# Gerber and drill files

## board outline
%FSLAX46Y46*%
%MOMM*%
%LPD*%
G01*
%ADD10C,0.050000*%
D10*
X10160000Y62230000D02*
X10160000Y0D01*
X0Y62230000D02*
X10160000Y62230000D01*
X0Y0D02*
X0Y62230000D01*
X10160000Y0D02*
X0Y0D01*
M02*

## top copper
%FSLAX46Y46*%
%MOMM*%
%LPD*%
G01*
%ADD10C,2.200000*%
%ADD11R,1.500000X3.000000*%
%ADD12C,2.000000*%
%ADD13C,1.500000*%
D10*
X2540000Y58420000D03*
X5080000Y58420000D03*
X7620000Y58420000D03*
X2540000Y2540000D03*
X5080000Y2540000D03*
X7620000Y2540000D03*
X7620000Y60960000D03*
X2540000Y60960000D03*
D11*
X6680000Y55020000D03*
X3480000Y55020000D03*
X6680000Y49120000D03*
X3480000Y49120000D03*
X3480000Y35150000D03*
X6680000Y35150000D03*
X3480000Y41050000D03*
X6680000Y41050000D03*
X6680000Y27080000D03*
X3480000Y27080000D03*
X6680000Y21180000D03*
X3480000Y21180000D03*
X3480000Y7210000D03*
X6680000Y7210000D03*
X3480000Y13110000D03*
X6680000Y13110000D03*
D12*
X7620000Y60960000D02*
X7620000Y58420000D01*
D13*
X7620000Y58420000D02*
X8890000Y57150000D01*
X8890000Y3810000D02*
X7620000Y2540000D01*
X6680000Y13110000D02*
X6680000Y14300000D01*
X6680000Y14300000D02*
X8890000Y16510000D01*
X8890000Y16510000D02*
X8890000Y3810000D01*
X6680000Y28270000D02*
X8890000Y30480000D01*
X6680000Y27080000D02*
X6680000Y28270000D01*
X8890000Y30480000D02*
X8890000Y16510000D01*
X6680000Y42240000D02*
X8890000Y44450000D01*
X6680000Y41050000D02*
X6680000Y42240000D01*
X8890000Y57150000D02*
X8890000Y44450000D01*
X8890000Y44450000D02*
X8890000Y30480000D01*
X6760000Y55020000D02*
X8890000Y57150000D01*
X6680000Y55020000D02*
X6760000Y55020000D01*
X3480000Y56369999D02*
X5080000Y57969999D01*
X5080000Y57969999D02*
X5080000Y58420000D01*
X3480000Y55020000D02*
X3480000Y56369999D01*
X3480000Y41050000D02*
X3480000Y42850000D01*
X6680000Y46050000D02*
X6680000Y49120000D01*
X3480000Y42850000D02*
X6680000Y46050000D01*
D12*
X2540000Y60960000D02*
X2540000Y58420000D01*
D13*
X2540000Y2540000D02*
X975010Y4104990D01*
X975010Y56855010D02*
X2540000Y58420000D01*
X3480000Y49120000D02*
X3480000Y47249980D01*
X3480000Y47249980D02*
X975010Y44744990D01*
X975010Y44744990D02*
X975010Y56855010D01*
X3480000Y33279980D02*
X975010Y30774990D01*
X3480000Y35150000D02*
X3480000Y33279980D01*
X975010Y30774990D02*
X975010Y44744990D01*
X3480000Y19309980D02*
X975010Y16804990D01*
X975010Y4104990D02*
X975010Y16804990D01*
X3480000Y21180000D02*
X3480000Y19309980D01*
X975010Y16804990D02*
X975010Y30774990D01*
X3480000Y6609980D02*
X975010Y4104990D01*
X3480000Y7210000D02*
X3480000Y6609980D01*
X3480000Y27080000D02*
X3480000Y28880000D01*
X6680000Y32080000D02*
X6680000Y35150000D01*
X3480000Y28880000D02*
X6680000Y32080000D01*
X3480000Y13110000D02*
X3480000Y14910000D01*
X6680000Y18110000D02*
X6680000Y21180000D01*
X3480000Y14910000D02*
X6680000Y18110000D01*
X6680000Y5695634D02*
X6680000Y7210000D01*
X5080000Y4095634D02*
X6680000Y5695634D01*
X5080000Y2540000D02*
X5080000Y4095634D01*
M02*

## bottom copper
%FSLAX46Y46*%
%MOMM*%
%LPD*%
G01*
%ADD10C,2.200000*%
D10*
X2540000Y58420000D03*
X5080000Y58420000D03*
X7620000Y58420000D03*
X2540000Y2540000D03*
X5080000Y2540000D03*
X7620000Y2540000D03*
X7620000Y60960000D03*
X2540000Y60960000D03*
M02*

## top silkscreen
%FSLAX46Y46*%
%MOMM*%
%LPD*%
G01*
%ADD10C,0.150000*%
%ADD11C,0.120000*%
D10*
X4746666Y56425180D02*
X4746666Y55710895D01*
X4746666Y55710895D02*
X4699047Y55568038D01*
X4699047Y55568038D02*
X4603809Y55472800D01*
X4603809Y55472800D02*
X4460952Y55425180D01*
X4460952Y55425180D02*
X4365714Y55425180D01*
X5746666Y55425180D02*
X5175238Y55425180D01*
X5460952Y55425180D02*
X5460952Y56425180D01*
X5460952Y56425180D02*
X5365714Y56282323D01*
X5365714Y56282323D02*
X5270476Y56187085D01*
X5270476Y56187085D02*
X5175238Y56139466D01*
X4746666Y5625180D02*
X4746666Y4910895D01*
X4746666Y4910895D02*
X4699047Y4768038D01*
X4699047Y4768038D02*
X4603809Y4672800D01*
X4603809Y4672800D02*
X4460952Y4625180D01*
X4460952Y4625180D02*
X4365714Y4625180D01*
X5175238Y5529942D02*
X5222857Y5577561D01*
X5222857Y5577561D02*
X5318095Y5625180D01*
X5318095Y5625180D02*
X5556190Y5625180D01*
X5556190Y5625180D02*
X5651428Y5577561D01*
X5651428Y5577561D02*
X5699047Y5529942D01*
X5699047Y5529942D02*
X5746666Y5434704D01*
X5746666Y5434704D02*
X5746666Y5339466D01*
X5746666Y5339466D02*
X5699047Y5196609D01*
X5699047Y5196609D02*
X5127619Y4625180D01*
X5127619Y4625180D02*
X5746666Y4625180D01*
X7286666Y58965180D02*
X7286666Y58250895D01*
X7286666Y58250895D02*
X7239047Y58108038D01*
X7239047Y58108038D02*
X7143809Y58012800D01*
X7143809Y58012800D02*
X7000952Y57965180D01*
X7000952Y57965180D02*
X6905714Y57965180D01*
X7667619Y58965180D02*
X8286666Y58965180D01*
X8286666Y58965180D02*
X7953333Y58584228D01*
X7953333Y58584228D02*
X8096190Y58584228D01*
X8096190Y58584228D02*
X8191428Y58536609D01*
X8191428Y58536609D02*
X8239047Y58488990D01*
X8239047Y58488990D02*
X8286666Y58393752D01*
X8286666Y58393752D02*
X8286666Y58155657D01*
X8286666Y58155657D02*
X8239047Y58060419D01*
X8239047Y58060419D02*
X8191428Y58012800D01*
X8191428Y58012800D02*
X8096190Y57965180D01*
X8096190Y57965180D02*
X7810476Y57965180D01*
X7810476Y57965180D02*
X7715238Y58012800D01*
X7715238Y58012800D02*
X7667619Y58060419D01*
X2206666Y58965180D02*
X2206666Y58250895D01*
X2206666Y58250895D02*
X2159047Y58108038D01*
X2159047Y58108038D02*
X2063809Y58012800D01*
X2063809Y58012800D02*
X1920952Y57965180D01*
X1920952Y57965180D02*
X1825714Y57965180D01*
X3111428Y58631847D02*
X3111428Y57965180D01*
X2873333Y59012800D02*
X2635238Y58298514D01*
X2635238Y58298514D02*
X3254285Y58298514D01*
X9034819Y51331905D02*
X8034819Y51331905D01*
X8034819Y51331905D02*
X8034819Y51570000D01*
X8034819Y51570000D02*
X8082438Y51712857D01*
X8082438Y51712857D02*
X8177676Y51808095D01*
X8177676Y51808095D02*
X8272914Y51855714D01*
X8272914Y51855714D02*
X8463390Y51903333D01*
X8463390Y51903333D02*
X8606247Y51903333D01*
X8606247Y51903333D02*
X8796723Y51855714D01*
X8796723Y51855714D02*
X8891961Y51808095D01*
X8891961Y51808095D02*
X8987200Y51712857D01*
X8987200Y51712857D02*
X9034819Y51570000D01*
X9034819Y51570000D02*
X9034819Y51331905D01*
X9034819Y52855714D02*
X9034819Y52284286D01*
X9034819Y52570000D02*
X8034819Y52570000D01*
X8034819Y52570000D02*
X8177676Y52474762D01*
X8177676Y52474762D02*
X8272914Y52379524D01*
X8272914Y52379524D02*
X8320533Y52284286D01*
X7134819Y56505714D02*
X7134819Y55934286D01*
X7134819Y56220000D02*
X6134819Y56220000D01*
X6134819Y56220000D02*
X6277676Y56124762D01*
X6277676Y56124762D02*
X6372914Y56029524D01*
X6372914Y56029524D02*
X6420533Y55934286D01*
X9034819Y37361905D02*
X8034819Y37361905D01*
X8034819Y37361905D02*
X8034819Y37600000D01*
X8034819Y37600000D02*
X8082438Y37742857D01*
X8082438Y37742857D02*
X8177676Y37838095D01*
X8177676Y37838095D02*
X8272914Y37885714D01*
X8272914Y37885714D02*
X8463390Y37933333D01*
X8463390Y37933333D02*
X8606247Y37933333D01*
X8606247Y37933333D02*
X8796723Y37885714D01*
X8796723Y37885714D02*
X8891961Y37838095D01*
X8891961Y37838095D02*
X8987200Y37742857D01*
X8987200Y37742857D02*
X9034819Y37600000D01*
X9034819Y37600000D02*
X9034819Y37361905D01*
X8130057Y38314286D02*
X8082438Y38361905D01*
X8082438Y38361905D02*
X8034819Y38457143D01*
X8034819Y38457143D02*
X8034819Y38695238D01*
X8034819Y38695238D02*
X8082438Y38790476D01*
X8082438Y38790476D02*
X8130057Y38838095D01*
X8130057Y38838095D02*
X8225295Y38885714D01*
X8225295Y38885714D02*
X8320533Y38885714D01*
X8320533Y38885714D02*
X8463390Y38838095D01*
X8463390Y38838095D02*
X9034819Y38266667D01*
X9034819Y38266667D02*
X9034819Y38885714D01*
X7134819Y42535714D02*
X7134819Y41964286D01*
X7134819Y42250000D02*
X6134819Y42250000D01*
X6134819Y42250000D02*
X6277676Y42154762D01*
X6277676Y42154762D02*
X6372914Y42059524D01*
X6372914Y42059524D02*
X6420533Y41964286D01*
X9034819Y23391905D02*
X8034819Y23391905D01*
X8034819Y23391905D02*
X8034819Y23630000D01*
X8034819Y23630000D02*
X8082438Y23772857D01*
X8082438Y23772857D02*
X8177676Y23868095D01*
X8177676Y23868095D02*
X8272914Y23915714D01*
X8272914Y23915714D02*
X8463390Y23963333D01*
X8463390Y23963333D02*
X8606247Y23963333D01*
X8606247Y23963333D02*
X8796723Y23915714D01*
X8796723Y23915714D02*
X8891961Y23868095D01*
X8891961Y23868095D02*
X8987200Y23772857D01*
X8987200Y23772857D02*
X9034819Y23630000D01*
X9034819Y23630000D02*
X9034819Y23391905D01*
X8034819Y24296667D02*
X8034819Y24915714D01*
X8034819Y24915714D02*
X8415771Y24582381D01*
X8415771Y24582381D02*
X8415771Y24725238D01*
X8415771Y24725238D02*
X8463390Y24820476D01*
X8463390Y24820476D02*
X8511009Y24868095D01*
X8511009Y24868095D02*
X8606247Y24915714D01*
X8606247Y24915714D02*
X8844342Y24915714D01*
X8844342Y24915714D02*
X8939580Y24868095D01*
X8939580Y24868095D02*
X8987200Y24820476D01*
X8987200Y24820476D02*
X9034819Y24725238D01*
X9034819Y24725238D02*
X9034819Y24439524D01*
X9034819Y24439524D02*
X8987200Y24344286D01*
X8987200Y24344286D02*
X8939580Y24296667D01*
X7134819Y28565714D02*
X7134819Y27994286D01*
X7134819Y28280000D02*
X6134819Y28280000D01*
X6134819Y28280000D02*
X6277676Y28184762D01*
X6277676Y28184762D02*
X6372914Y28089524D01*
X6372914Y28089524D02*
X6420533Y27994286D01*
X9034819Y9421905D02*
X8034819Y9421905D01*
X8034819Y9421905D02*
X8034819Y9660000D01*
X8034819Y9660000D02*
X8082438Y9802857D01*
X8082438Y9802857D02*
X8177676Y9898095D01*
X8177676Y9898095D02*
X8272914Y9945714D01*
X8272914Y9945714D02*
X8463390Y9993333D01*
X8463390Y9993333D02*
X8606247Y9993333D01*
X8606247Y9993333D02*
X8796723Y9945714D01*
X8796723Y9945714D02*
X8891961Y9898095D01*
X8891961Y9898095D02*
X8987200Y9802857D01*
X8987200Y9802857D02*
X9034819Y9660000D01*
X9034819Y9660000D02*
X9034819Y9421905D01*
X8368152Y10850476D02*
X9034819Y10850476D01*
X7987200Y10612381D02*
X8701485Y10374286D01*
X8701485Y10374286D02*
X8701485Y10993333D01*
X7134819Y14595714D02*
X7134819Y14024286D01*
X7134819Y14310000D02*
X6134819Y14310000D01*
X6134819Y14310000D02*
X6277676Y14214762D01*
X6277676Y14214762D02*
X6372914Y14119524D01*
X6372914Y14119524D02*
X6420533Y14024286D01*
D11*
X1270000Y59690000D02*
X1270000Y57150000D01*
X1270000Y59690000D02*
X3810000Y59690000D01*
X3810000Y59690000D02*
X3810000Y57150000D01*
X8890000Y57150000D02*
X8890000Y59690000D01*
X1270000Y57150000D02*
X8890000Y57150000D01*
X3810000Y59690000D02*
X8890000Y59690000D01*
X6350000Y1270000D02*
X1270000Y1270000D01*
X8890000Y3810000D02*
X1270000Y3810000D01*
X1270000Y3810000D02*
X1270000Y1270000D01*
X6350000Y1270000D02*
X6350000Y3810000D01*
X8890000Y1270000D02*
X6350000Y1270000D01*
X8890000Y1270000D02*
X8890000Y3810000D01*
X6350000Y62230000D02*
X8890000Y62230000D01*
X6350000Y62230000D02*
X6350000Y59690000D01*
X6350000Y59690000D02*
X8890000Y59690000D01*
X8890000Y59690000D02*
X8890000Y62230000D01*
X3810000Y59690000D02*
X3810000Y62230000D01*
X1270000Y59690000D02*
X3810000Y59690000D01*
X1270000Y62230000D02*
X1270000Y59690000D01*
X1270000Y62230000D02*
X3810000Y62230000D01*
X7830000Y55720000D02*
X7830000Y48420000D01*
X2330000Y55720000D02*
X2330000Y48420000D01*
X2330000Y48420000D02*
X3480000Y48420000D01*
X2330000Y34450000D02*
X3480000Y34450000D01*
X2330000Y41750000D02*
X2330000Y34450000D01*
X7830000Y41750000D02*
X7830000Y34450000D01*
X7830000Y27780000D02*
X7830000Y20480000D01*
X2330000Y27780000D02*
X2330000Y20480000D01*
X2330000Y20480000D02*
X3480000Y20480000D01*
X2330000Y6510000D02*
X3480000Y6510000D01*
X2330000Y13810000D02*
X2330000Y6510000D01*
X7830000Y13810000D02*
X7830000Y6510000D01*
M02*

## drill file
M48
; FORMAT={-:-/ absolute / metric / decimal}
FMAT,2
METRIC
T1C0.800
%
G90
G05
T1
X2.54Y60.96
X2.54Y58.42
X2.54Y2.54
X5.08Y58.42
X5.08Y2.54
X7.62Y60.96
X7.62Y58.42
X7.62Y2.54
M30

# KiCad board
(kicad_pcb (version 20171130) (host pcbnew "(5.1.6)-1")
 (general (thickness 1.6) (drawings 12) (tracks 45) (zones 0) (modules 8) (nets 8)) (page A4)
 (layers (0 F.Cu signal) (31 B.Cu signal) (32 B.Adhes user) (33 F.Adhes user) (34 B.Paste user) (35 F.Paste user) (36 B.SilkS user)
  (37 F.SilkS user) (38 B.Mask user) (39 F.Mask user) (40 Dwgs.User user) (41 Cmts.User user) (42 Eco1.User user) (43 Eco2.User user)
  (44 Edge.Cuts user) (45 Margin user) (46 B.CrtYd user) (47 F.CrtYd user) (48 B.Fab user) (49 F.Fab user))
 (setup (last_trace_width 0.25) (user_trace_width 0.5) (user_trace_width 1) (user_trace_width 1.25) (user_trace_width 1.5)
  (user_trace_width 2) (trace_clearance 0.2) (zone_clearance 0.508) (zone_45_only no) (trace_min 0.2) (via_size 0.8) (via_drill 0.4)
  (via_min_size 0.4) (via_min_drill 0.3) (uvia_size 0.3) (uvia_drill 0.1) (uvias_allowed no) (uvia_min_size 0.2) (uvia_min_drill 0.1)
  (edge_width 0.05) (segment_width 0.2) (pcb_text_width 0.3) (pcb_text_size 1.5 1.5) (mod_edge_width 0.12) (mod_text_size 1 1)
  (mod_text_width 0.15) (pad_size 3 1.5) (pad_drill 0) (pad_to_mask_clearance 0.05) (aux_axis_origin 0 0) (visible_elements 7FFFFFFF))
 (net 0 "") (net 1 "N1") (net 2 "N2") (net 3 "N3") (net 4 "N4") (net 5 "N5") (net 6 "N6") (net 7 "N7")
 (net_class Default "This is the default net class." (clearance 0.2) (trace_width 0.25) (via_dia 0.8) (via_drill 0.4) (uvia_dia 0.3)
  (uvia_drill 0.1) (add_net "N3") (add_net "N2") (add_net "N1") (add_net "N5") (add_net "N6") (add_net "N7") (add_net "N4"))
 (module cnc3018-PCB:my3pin (layer F.Cu) (at 5.08 -58.42)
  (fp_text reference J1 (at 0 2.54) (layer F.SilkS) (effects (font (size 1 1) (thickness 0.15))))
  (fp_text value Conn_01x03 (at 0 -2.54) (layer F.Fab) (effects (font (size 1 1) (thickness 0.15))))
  (fp_line (start -3.81 -1.27) (end -3.81 1.27) (layer F.SilkS) (width 0.12))
  (fp_line (start -3.81 -1.27) (end -1.27 -1.27) (layer F.SilkS) (width 0.12))
  (fp_line (start -1.27 -1.27) (end -1.27 1.27) (layer F.SilkS) (width 0.12))
  (fp_line (start 3.81 1.27) (end 3.81 -1.27) (layer F.SilkS) (width 0.12))
  (fp_line (start -3.81 1.27) (end 3.81 1.27) (layer F.SilkS) (width 0.12))
  (fp_line (start -1.27 -1.27) (end 3.81 -1.27) (layer F.SilkS) (width 0.12))
  (pad 1 thru_hole circle (at -2.54 0) (size 2.2 2.2) (drill 0.8) (layers *.Cu *.Mask) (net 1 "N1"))
  (pad 2 thru_hole circle (at 0 0) (size 2.2 2.2) (drill 0.8) (layers *.Cu *.Mask) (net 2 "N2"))
  (pad 3 thru_hole circle (at 2.54 0) (size 2.2 2.2) (drill 0.8) (layers *.Cu *.Mask) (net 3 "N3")))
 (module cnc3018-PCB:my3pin (layer F.Cu) (at 5.08 -2.54 180)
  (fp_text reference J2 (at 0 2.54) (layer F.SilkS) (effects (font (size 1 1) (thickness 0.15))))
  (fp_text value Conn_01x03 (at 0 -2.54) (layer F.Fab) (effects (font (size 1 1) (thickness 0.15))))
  (fp_line (start -1.27 -1.27) (end 3.81 -1.27) (layer F.SilkS) (width 0.12))
  (fp_line (start -3.81 1.27) (end 3.81 1.27) (layer F.SilkS) (width 0.12))
  (fp_line (start 3.81 1.27) (end 3.81 -1.27) (layer F.SilkS) (width 0.12))
  (fp_line (start -1.27 -1.27) (end -1.27 1.27) (layer F.SilkS) (width 0.12))
  (fp_line (start -3.81 -1.27) (end -1.27 -1.27) (layer F.SilkS) (width 0.12))
  (fp_line (start -3.81 -1.27) (end -3.81 1.27) (layer F.SilkS) (width 0.12))
  (pad 3 thru_hole circle (at 2.54 0 180) (size 2.2 2.2) (drill 0.8) (layers *.Cu *.Mask) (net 1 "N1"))
  (pad 2 thru_hole circle (at 0 0 180) (size 2.2 2.2) (drill 0.8) (layers *.Cu *.Mask) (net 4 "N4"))
  (pad 1 thru_hole circle (at -2.54 0 180) (size 2.2 2.2) (drill 0.8) (layers *.Cu *.Mask) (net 3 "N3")))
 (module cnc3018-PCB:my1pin (layer F.Cu) (at 7.62 -60.96)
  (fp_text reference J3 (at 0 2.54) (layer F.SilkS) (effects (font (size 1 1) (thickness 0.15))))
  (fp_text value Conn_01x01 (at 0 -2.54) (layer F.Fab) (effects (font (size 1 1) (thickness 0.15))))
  (fp_line (start -1.27 -1.27) (end 1.27 -1.27) (layer F.SilkS) (width 0.12))
  (fp_line (start -1.27 -1.27) (end -1.27 1.27) (layer F.SilkS) (width 0.12))
  (fp_line (start -1.27 1.27) (end 1.27 1.27) (layer F.SilkS) (width 0.12))
  (fp_line (start 1.27 1.27) (end 1.27 -1.27) (layer F.SilkS) (width 0.12))
  (pad 1 thru_hole circle (at 0 0) (size 2.2 2.2) (drill 0.8) (layers *.Cu *.Mask) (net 3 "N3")))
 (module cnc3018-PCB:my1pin (layer F.Cu) (at 2.54 -60.96)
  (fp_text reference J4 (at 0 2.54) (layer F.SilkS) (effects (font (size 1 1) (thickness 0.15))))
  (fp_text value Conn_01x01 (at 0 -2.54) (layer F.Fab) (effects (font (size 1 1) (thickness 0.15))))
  (fp_line (start 1.27 1.27) (end 1.27 -1.27) (layer F.SilkS) (width 0.12))
  (fp_line (start -1.27 1.27) (end 1.27 1.27) (layer F.SilkS) (width 0.12))
  (fp_line (start -1.27 -1.27) (end -1.27 1.27) (layer F.SilkS) (width 0.12))
  (fp_line (start -1.27 -1.27) (end 1.27 -1.27) (layer F.SilkS) (width 0.12))
  (pad 1 thru_hole circle (at 0 0) (size 2.2 2.2) (drill 0.8) (layers *.Cu *.Mask) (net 1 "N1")))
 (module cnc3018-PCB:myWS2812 (layer F.Cu) (at 5.08 -52.07 270)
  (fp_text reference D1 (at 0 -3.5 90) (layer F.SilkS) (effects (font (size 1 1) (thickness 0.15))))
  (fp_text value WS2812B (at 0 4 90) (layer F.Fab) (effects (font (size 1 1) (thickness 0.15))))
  (fp_line (start -3.65 -2.75) (end 3.65 -2.75) (layer F.SilkS) (width 0.12))
  (fp_line (start -3.65 2.75) (end 3.65 2.75) (layer F.SilkS) (width 0.12))
  (fp_line (start 3.65 2.75) (end 3.65 1.6) (layer F.SilkS) (width 0.12))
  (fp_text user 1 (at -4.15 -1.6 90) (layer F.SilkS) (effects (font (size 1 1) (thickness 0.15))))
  (pad 1 smd rect (at -2.95 -1.6 270) (size 3 1.5) (layers F.Cu F.Paste F.Mask) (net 3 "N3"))
  (pad 2 smd rect (at -2.95 1.6 270) (size 3 1.5) (layers F.Cu F.Paste F.Mask) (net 2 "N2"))
  (pad 4 smd rect (at 2.95 -1.6 270) (size 3 1.5) (layers F.Cu F.Paste F.Mask) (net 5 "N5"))
  (pad 3 smd rect (at 2.95 1.6 270) (size 3 1.5) (layers F.Cu F.Paste F.Mask) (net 1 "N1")))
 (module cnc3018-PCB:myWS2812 (layer F.Cu) (at 5.08 -38.1 270)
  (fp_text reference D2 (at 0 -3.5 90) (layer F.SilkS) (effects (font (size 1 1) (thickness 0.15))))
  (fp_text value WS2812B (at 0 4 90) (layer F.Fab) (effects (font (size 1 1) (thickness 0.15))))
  (fp_line (start 3.65 2.75) (end 3.65 1.6) (layer F.SilkS) (width 0.12))
  (fp_line (start -3.65 2.75) (end 3.65 2.75) (layer F.SilkS) (width 0.12))
  (fp_line (start -3.65 -2.75) (end 3.65 -2.75) (layer F.SilkS) (width 0.12))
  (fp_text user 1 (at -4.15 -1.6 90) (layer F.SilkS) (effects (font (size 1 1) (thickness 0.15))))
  (pad 3 smd rect (at 2.95 1.6 270) (size 3 1.5) (layers F.Cu F.Paste F.Mask) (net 1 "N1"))
  (pad 4 smd rect (at 2.95 -1.6 270) (size 3 1.5) (layers F.Cu F.Paste F.Mask) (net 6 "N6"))
  (pad 2 smd rect (at -2.95 1.6 270) (size 3 1.5) (layers F.Cu F.Paste F.Mask) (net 5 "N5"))
  (pad 1 smd rect (at -2.95 -1.6 270) (size 3 1.5) (layers F.Cu F.Paste F.Mask) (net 3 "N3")))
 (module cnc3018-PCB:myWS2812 (layer F.Cu) (at 5.08 -24.13 270)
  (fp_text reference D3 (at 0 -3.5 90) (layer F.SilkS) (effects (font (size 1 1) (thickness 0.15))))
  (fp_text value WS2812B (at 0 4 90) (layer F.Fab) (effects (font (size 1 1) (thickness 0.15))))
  (fp_line (start -3.65 -2.75) (end 3.65 -2.75) (layer F.SilkS) (width 0.12))
  (fp_line (start -3.65 2.75) (end 3.65 2.75) (layer F.SilkS) (width 0.12))
  (fp_line (start 3.65 2.75) (end 3.65 1.6) (layer F.SilkS) (width 0.12))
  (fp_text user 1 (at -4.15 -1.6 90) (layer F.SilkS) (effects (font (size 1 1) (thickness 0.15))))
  (pad 1 smd rect (at -2.95 -1.6 270) (size 3 1.5) (layers F.Cu F.Paste F.Mask) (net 3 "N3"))
  (pad 2 smd rect (at -2.95 1.6 270) (size 3 1.5) (layers F.Cu F.Paste F.Mask) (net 6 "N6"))
  (pad 4 smd rect (at 2.95 -1.6 270) (size 3 1.5) (layers F.Cu F.Paste F.Mask) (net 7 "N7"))
  (pad 3 smd rect (at 2.95 1.6 270) (size 3 1.5) (layers F.Cu F.Paste F.Mask) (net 1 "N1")))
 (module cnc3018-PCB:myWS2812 (layer F.Cu) (at 5.08 -10.16 270)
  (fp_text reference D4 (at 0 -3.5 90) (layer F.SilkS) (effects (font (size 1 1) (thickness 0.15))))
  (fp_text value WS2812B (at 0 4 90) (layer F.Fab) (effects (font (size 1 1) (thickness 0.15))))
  (fp_line (start 3.65 2.75) (end 3.65 1.6) (layer F.SilkS) (width 0.12))
  (fp_line (start -3.65 2.75) (end 3.65 2.75) (layer F.SilkS) (width 0.12))
  (fp_line (start -3.65 -2.75) (end 3.65 -2.75) (layer F.SilkS) (width 0.12))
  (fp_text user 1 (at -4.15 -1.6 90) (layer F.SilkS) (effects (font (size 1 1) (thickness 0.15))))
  (pad 3 smd rect (at 2.95 1.6 270) (size 3 1.5) (layers F.Cu F.Paste F.Mask) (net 1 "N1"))
  (pad 4 smd rect (at 2.95 -1.6 270) (size 3 1.5) (layers F.Cu F.Paste F.Mask) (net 4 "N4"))
  (pad 2 smd rect (at -2.95 1.6 270) (size 3 1.5) (layers F.Cu F.Paste F.Mask) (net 7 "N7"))
  (pad 1 smd rect (at -2.95 -1.6 270) (size 3 1.5) (layers F.Cu F.Paste F.Mask) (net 3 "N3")))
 (gr_line (start 10.16 -62.23) (end 10.16 0) (layer Edge.Cuts) (width 0.05))
 (gr_line (start 0 -62.23) (end 10.16 -62.23) (layer Edge.Cuts) (width 0.05))
 (gr_line (start 0 0) (end 0 -62.23) (layer Edge.Cuts) (width 0.05))
 (gr_line (start 10.16 0) (end 0 0) (layer Edge.Cuts) (width 0.05))
 (segment (start 7.62 -60.96) (end 7.62 -58.42) (width 2) (layer F.Cu) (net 3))
 (segment (start 7.62 -58.42) (end 8.89 -57.15) (width 1.5) (layer F.Cu) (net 3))
 (segment (start 8.89 -3.81) (end 7.62 -2.54) (width 1.5) (layer F.Cu) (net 3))
 (segment (start 6.68 -13.11) (end 6.68 -14.3) (width 1.5) (layer F.Cu) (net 3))
 (segment (start 6.68 -14.3) (end 8.89 -16.51) (width 1.5) (layer F.Cu) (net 3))
 (segment (start 8.89 -16.51) (end 8.89 -3.81) (width 1.5) (layer F.Cu) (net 3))
 (segment (start 6.68 -28.27) (end 8.89 -30.48) (width 1.5) (layer F.Cu) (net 3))
 (segment (start 6.68 -27.08) (end 6.68 -28.27) (width 1.5) (layer F.Cu) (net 3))
 (segment (start 8.89 -30.48) (end 8.89 -16.51) (width 1.5) (layer F.Cu) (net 3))
 (segment (start 6.68 -42.24) (end 8.89 -44.45) (width 1.5) (layer F.Cu) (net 3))
 (segment (start 6.68 -41.05) (end 6.68 -42.24) (width 1.5) (layer F.Cu) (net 3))
 (segment (start 8.89 -57.15) (end 8.89 -44.45) (width 1.5) (layer F.Cu) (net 3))
 (segment (start 8.89 -44.45) (end 8.89 -30.48) (width 1.5) (layer F.Cu) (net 3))
 (segment (start 6.76 -55.02) (end 8.89 -57.15) (width 1.5) (layer F.Cu) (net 3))
 (segment (start 6.68 -55.02) (end 6.76 -55.02) (width 1.5) (layer F.Cu) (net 3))
 (segment (start 3.48 -56.369999) (end 5.08 -57.969999) (width 1.5) (layer F.Cu) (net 2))
 (segment (start 5.08 -57.969999) (end 5.08 -58.42) (width 1.5) (layer F.Cu) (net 2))
 (segment (start 3.48 -55.02) (end 3.48 -56.369999) (width 1.5) (layer F.Cu) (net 2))
 (segment (start 3.48 -41.05) (end 3.48 -42.85) (width 1.5) (layer F.Cu) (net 5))
 (segment (start 6.68 -46.05) (end 6.68 -49.12) (width 1.5) (layer F.Cu) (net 5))
 (segment (start 3.48 -42.85) (end 6.68 -46.05) (width 1.5) (layer F.Cu) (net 5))
 (segment (start 2.54 -60.96) (end 2.54 -58.42) (width 2) (layer F.Cu) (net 1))
 (segment (start 2.54 -2.54) (end 0.97501 -4.10499) (width 1.5) (layer F.Cu) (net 1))
 (segment (start 0.97501 -56.85501) (end 2.54 -58.42) (width 1.5) (layer F.Cu) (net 1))
 (segment (start 3.48 -49.12) (end 3.48 -47.24998) (width 1.5) (layer F.Cu) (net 1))
 (segment (start 3.48 -47.24998) (end 0.97501 -44.74499) (width 1.5) (layer F.Cu) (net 1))
 (segment (start 0.97501 -44.74499) (end 0.97501 -56.85501) (width 1.5) (layer F.Cu) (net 1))
 (segment (start 3.48 -33.27998) (end 0.97501 -30.77499) (width 1.5) (layer F.Cu) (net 1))
 (segment (start 3.48 -35.15) (end 3.48 -33.27998) (width 1.5) (layer F.Cu) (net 1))
 (segment (start 0.97501 -30.77499) (end 0.97501 -44.74499) (width 1.5) (layer F.Cu) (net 1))
 (segment (start 3.48 -19.30998) (end 0.97501 -16.80499) (width 1.5) (layer F.Cu) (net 1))
 (segment (start 0.97501 -4.10499) (end 0.97501 -16.80499) (width 1.5) (layer F.Cu) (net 1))
 (segment (start 3.48 -21.18) (end 3.48 -19.30998) (width 1.5) (layer F.Cu) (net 1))
 (segment (start 0.97501 -16.80499) (end 0.97501 -30.77499) (width 1.5) (layer F.Cu) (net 1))
 (segment (start 3.48 -6.60998) (end 0.97501 -4.10499) (width 1.5) (layer F.Cu) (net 1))
 (segment (start 3.48 -7.21) (end 3.48 -6.60998) (width 1.5) (layer F.Cu) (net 1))
 (segment (start 3.48 -27.08) (end 3.48 -28.88) (width 1.5) (layer F.Cu) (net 6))
 (segment (start 6.68 -32.08) (end 6.68 -35.15) (width 1.5) (layer F.Cu) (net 6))
 (segment (start 3.48 -28.88) (end 6.68 -32.08) (width 1.5) (layer F.Cu) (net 6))
 (segment (start 3.48 -13.11) (end 3.48 -14.91) (width 1.5) (layer F.Cu) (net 7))
 (segment (start 6.68 -18.11) (end 6.68 -21.18) (width 1.5) (layer F.Cu) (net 7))
 (segment (start 3.48 -14.91) (end 6.68 -18.11) (width 1.5) (layer F.Cu) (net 7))
 (segment (start 6.68 -5.695634) (end 6.68 -7.21) (width 1.5) (layer F.Cu) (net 4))
 (segment (start 5.08 -4.095634) (end 6.68 -5.695634) (width 1.5) (layer F.Cu) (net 4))
 (segment (start 5.08 -2.54) (end 5.08 -4.095634) (width 1.5) (layer F.Cu) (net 4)))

